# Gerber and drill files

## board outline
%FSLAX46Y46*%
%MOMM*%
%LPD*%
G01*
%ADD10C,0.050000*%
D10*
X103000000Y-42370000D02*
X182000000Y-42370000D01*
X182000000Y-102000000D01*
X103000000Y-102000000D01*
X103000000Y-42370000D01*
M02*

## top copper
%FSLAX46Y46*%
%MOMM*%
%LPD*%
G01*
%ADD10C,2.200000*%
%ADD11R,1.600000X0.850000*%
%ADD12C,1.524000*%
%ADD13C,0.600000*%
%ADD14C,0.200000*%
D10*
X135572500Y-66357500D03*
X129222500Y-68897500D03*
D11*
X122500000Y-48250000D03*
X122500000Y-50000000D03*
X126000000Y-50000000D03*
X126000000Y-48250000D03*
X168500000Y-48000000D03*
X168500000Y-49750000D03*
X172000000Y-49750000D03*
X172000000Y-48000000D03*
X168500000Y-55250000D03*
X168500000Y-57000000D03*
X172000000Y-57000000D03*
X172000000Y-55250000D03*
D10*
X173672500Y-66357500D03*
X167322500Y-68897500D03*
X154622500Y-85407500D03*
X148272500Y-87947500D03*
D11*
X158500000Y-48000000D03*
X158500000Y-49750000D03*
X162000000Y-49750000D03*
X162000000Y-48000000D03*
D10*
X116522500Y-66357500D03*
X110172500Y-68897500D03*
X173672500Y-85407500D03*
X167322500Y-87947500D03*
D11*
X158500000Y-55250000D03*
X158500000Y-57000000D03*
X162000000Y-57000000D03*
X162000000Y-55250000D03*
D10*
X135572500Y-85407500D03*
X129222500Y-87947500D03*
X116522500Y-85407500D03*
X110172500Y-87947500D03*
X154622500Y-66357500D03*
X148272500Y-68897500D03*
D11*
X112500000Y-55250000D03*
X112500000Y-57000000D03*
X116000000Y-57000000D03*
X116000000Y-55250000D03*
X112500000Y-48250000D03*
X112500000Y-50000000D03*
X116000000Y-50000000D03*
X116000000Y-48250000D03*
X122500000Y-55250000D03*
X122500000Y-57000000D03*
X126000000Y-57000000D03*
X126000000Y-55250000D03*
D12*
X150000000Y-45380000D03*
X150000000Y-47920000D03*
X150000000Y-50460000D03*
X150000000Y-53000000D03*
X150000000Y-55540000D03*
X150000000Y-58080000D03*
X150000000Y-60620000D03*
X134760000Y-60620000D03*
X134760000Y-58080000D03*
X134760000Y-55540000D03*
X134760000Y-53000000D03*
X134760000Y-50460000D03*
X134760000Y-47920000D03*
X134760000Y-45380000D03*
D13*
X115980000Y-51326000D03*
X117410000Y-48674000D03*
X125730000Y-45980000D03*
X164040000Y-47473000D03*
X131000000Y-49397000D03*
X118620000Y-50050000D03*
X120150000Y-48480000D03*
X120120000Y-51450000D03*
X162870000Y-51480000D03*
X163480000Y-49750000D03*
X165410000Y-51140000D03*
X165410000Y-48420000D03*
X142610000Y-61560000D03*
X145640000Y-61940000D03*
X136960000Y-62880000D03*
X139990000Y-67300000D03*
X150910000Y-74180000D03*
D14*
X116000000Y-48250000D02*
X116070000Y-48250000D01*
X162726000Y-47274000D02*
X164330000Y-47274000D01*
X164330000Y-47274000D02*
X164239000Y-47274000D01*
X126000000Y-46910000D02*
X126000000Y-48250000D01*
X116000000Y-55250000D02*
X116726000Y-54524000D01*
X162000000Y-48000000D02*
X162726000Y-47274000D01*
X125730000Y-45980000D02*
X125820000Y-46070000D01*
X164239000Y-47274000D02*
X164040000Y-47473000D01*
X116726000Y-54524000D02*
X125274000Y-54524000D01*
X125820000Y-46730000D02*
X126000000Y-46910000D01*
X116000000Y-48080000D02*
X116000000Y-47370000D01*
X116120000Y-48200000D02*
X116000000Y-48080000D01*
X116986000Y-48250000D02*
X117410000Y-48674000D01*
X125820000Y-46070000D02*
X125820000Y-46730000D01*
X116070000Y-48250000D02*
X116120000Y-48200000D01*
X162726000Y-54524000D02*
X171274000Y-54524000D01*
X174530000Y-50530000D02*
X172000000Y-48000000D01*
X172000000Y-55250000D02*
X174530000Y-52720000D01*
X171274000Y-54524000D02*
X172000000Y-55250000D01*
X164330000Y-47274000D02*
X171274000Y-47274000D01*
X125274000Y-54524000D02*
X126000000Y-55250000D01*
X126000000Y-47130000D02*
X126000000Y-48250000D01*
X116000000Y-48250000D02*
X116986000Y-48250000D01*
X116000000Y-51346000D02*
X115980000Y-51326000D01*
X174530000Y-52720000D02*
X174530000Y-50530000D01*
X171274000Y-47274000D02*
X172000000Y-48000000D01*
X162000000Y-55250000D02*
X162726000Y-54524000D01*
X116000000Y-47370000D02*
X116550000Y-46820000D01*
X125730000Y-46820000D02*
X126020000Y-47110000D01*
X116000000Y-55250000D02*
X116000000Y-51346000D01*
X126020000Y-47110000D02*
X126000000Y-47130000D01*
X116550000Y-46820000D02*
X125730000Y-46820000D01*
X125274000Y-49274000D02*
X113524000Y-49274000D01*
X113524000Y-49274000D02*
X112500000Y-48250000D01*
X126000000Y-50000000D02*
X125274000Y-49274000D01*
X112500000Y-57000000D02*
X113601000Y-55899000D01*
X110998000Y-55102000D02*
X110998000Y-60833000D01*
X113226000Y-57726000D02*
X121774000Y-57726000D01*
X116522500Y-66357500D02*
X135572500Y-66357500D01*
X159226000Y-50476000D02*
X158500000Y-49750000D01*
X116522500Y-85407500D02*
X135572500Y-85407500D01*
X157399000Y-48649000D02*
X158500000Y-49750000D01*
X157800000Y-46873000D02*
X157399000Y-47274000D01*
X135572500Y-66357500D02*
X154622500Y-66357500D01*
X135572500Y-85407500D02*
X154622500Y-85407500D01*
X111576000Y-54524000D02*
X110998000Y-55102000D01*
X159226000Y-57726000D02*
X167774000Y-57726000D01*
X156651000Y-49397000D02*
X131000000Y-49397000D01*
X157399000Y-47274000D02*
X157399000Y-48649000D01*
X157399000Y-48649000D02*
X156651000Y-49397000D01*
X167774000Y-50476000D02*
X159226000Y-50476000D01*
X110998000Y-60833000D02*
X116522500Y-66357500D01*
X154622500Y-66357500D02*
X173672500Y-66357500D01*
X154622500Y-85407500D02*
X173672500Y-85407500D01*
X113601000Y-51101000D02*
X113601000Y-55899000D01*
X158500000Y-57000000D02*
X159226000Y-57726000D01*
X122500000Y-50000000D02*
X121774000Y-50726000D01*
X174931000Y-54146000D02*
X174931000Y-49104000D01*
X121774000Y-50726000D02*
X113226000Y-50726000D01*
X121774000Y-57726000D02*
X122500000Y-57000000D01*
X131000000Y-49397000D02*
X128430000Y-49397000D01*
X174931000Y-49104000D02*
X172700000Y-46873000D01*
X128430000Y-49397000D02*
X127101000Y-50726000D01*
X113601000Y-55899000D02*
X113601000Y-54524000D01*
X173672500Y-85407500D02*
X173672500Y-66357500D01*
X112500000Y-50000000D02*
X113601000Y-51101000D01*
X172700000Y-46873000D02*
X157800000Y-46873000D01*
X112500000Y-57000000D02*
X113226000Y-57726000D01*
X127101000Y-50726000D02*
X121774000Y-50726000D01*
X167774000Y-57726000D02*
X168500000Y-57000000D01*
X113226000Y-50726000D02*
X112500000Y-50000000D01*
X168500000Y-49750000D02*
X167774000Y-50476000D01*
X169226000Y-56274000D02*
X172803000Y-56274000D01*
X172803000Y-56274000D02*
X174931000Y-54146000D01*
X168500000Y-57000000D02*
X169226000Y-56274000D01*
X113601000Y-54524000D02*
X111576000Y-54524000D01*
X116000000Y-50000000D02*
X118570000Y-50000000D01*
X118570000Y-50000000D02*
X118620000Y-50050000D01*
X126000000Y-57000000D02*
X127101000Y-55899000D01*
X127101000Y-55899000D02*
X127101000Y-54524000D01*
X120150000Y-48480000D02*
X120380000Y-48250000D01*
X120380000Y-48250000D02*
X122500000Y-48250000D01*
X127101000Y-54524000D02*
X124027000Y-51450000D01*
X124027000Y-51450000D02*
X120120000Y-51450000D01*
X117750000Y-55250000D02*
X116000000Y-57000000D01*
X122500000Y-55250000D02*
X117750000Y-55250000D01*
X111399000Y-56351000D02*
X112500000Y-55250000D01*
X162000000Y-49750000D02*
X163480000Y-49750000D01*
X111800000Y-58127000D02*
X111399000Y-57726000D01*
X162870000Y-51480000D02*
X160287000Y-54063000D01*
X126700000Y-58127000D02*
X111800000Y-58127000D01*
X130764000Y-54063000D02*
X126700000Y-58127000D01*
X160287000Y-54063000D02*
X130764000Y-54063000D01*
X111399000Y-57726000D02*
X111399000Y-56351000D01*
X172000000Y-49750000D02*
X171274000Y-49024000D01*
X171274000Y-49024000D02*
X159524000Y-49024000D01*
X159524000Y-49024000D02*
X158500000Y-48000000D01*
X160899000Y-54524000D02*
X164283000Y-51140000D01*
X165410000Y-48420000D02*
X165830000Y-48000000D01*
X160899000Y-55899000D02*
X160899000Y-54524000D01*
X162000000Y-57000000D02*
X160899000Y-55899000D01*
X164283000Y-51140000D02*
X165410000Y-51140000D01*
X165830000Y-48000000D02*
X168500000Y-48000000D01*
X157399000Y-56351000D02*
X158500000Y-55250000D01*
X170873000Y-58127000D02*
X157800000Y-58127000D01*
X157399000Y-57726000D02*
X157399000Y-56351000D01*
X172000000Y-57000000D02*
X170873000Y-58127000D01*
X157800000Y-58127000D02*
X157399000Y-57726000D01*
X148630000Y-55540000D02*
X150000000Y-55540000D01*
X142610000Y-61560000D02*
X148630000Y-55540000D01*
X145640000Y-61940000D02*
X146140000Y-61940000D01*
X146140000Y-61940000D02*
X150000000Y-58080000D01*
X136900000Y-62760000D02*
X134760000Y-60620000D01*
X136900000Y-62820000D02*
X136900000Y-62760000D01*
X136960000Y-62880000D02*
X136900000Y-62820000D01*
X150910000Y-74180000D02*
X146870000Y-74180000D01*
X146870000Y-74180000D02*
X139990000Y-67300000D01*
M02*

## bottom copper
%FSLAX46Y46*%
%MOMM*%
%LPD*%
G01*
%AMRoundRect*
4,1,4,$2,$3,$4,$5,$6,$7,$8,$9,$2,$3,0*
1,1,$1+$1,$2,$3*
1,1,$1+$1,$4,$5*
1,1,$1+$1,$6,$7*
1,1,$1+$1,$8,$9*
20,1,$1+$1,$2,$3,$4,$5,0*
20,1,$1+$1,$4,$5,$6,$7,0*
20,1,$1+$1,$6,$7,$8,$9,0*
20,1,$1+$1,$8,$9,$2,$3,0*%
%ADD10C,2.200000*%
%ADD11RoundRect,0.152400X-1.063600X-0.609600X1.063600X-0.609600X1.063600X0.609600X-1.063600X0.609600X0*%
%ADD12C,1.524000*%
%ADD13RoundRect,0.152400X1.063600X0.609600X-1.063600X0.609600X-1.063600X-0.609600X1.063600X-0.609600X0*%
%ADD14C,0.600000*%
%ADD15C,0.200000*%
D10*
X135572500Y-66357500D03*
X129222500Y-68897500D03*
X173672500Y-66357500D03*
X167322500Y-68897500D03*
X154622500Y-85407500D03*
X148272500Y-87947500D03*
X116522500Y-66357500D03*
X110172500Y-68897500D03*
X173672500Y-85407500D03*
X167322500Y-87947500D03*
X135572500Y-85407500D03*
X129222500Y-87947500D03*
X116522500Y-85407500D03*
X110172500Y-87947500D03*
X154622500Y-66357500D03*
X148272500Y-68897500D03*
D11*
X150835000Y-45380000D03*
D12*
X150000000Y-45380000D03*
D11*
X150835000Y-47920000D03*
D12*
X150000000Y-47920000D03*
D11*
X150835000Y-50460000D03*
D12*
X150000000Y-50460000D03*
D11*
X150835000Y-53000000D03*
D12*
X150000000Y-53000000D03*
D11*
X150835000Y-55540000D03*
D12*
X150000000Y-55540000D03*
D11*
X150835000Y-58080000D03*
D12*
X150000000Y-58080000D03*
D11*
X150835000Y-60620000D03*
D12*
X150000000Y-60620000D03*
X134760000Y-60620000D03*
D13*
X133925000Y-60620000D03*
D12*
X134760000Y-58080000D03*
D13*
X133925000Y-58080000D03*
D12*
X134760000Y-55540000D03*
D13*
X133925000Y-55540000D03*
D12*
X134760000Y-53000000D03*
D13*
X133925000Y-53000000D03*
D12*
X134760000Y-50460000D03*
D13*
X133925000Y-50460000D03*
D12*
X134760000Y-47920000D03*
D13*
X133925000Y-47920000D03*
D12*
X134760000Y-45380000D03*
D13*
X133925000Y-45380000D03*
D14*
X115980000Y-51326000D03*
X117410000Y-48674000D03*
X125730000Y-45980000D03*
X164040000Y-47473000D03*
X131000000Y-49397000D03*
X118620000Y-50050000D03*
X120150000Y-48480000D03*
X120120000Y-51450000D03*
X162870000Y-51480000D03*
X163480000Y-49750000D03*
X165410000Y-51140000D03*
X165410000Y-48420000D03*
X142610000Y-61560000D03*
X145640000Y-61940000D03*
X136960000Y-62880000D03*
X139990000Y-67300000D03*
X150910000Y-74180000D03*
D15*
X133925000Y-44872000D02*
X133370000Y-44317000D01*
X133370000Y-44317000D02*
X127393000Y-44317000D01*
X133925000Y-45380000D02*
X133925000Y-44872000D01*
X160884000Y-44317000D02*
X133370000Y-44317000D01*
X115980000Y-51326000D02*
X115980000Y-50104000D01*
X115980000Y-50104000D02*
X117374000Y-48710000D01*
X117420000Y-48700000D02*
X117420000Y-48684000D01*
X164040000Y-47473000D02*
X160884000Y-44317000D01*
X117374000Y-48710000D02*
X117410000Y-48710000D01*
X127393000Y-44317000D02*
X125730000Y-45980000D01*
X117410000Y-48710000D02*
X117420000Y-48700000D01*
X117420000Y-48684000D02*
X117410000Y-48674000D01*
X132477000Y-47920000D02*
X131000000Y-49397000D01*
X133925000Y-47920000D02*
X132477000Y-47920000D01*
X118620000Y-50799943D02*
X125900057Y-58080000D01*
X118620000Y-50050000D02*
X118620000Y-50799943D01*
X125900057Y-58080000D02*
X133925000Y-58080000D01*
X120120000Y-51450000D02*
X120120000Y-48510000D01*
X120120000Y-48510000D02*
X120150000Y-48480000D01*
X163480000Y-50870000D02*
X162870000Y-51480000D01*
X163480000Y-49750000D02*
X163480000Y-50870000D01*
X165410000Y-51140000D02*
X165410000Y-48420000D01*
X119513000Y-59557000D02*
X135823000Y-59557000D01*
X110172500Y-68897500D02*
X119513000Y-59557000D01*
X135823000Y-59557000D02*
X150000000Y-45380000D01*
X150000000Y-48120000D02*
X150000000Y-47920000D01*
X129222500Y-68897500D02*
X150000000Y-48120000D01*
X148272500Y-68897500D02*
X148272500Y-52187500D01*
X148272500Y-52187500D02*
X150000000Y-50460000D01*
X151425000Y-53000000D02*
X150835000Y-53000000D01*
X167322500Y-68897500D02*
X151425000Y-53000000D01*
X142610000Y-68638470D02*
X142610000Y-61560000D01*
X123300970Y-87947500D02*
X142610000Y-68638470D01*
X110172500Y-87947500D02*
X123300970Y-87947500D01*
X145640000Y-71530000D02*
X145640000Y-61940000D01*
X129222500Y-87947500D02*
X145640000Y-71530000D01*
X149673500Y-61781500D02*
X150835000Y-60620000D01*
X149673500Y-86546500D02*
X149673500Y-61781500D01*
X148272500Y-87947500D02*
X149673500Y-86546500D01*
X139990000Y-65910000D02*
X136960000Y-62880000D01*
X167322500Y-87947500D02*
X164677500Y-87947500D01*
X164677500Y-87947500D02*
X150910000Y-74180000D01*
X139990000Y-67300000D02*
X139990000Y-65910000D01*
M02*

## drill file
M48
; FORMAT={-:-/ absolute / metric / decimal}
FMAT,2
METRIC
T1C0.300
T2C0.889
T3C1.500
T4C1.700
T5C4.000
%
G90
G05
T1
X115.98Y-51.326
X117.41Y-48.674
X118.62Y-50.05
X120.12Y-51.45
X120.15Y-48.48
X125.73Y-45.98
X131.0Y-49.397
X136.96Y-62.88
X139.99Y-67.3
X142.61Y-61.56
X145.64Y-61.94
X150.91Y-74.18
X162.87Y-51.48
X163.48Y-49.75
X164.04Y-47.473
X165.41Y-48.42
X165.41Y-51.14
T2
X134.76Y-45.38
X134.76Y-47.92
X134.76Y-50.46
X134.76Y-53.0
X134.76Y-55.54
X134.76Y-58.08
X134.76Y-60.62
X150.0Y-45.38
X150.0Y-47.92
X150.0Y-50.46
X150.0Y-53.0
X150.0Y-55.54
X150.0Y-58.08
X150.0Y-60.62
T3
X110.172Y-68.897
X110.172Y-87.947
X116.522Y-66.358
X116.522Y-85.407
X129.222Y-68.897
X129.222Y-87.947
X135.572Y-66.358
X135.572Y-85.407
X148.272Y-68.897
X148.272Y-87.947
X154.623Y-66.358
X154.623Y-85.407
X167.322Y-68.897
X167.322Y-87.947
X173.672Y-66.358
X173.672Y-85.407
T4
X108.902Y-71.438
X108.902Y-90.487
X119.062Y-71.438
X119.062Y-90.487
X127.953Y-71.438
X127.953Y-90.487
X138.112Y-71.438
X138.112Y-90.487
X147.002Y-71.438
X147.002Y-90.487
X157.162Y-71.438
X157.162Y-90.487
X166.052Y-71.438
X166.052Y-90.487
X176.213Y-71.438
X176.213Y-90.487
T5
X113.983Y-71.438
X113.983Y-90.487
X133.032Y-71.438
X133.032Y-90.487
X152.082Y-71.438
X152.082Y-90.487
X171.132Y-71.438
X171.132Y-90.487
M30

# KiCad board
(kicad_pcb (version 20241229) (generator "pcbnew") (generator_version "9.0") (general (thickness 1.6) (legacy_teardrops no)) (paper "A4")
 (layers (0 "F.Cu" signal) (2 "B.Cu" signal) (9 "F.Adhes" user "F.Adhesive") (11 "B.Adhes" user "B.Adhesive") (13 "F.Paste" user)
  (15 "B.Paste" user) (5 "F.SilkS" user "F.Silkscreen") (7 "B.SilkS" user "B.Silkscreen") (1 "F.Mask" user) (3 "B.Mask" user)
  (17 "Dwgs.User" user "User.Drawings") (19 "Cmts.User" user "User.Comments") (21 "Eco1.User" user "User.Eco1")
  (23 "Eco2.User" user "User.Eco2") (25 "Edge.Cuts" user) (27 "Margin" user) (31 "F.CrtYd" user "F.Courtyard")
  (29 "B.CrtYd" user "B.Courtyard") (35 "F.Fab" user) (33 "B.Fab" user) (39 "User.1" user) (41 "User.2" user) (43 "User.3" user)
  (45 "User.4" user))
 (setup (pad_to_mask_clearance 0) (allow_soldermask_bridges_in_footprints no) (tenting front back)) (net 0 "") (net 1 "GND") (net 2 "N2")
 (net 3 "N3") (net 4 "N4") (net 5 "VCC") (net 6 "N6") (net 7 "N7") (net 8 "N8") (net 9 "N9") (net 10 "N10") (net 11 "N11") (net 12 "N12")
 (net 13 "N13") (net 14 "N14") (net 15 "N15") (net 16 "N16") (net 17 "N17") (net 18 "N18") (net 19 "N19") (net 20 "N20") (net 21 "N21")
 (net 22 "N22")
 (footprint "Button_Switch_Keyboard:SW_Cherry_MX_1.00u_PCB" (layer "F.Cu") (at 135.5725 66.3575)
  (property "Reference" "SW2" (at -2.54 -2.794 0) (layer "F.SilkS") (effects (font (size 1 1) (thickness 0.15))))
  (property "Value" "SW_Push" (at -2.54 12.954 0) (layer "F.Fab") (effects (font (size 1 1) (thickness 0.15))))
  (pad "" np_thru_hole circle (at -7.62 5.08) (size 1.7 1.7) (drill 1.7) (layers "*.Cu" "*.Mask"))
  (pad "" np_thru_hole circle (at -2.54 5.08) (size 4 4) (drill 4) (layers "*.Cu" "*.Mask"))
  (pad "" np_thru_hole circle (at 2.54 5.08) (size 1.7 1.7) (drill 1.7) (layers "*.Cu" "*.Mask"))
  (pad "1" thru_hole circle (at 0 0) (size 2.2 2.2) (drill 1.5) (layers "*.Cu" "*.Mask") (remove_unused_layers no) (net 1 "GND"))
  (pad "2" thru_hole circle (at -6.35 2.54) (size 2.2 2.2) (drill 1.5) (layers "*.Cu" "*.Mask") (remove_unused_layers no) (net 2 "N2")))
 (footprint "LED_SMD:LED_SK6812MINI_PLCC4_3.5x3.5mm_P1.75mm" (layer "F.Cu") (at 124.25 49.125)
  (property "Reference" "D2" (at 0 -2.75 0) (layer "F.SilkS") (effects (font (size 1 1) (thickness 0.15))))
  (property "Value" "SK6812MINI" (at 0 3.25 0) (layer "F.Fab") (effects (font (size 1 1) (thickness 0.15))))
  (pad "1" smd rect (at -1.75 -0.875) (size 1.6 0.85) (layers "F.Cu" "F.Mask" "F.Paste") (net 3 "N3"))
  (pad "2" smd rect (at -1.75 0.875) (size 1.6 0.85) (layers "F.Cu" "F.Mask" "F.Paste") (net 1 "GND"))
  (pad "3" smd rect (at 1.75 0.875) (size 1.6 0.85) (layers "F.Cu" "F.Mask" "F.Paste") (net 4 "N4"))
  (pad "4" smd rect (at 1.75 -0.875) (size 1.6 0.85) (layers "F.Cu" "F.Mask" "F.Paste") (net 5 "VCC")))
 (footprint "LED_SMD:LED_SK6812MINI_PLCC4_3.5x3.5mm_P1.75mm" (layer "F.Cu") (at 170.25 48.875)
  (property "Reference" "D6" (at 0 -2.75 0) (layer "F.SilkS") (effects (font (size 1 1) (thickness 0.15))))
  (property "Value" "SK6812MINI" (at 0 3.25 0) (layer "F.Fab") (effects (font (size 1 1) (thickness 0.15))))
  (pad "1" smd rect (at -1.75 -0.875) (size 1.6 0.85) (layers "F.Cu" "F.Mask" "F.Paste") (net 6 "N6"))
  (pad "2" smd rect (at -1.75 0.875) (size 1.6 0.85) (layers "F.Cu" "F.Mask" "F.Paste") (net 1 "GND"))
  (pad "3" smd rect (at 1.75 0.875) (size 1.6 0.85) (layers "F.Cu" "F.Mask" "F.Paste") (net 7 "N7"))
  (pad "4" smd rect (at 1.75 -0.875) (size 1.6 0.85) (layers "F.Cu" "F.Mask" "F.Paste") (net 5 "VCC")))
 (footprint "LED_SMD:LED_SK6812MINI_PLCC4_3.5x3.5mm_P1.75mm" (layer "F.Cu") (at 170.25 56.125)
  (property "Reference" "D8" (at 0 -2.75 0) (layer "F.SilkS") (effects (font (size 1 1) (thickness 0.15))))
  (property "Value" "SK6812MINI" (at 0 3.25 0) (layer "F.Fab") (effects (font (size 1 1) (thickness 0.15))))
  (pad "1" smd rect (at -1.75 -0.875) (size 1.6 0.85) (layers "F.Cu" "F.Mask" "F.Paste") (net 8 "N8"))
  (pad "2" smd rect (at -1.75 0.875) (size 1.6 0.85) (layers "F.Cu" "F.Mask" "F.Paste") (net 1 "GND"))
  (pad "3" smd rect (at 1.75 0.875) (size 1.6 0.85) (layers "F.Cu" "F.Mask" "F.Paste") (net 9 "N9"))
  (pad "4" smd rect (at 1.75 -0.875) (size 1.6 0.85) (layers "F.Cu" "F.Mask" "F.Paste") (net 5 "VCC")))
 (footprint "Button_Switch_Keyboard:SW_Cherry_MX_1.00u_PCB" (layer "F.Cu") (at 173.6725 66.3575)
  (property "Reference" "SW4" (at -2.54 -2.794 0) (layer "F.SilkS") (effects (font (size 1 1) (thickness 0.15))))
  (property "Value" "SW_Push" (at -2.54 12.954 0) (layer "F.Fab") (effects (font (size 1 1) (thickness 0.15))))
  (pad "" np_thru_hole circle (at -7.62 5.08) (size 1.7 1.7) (drill 1.7) (layers "*.Cu" "*.Mask"))
  (pad "" np_thru_hole circle (at -2.54 5.08) (size 4 4) (drill 4) (layers "*.Cu" "*.Mask"))
  (pad "" np_thru_hole circle (at 2.54 5.08) (size 1.7 1.7) (drill 1.7) (layers "*.Cu" "*.Mask"))
  (pad "1" thru_hole circle (at 0 0) (size 2.2 2.2) (drill 1.5) (layers "*.Cu" "*.Mask") (remove_unused_layers no) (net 1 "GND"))
  (pad "2" thru_hole circle (at -6.35 2.54) (size 2.2 2.2) (drill 1.5) (layers "*.Cu" "*.Mask") (remove_unused_layers no) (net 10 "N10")))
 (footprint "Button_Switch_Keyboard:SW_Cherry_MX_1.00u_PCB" (layer "F.Cu") (at 154.6225 85.4075)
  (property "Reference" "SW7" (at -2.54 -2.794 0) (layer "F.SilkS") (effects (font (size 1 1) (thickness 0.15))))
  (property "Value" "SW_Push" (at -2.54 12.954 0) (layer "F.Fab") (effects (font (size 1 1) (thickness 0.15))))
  (pad "" np_thru_hole circle (at -7.62 5.08) (size 1.7 1.7) (drill 1.7) (layers "*.Cu" "*.Mask"))
  (pad "" np_thru_hole circle (at -2.54 5.08) (size 4 4) (drill 4) (layers "*.Cu" "*.Mask"))
  (pad "" np_thru_hole circle (at 2.54 5.08) (size 1.7 1.7) (drill 1.7) (layers "*.Cu" "*.Mask"))
  (pad "1" thru_hole circle (at 0 0) (size 2.2 2.2) (drill 1.5) (layers "*.Cu" "*.Mask") (remove_unused_layers no) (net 1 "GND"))
  (pad "2" thru_hole circle (at -6.35 2.54) (size 2.2 2.2) (drill 1.5) (layers "*.Cu" "*.Mask") (remove_unused_layers no) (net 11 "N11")))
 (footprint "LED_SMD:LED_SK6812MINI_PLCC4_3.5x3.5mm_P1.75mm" (layer "F.Cu") (at 160.25 48.875)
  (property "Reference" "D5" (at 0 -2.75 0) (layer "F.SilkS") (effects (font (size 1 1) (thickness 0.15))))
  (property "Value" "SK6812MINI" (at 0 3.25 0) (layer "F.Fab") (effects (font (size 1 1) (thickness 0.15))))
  (pad "1" smd rect (at -1.75 -0.875) (size 1.6 0.85) (layers "F.Cu" "F.Mask" "F.Paste") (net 7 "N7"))
  (pad "2" smd rect (at -1.75 0.875) (size 1.6 0.85) (layers "F.Cu" "F.Mask" "F.Paste") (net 1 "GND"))
  (pad "3" smd rect (at 1.75 0.875) (size 1.6 0.85) (layers "F.Cu" "F.Mask" "F.Paste") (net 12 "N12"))
  (pad "4" smd rect (at 1.75 -0.875) (size 1.6 0.85) (layers "F.Cu" "F.Mask" "F.Paste") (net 5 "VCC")))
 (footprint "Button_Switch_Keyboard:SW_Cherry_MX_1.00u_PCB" (layer "F.Cu") (at 116.5225 66.3575)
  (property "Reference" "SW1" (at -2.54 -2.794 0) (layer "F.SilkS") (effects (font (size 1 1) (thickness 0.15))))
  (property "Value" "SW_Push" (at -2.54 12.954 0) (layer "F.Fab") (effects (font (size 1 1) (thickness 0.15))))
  (pad "" np_thru_hole circle (at -7.62 5.08) (size 1.7 1.7) (drill 1.7) (layers "*.Cu" "*.Mask"))
  (pad "" np_thru_hole circle (at -2.54 5.08) (size 4 4) (drill 4) (layers "*.Cu" "*.Mask"))
  (pad "" np_thru_hole circle (at 2.54 5.08) (size 1.7 1.7) (drill 1.7) (layers "*.Cu" "*.Mask"))
  (pad "1" thru_hole circle (at 0 0) (size 2.2 2.2) (drill 1.5) (layers "*.Cu" "*.Mask") (remove_unused_layers no) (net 1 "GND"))
  (pad "2" thru_hole circle (at -6.35 2.54) (size 2.2 2.2) (drill 1.5) (layers "*.Cu" "*.Mask") (remove_unused_layers no) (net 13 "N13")))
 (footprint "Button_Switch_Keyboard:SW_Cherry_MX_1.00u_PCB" (layer "F.Cu") (at 173.6725 85.4075)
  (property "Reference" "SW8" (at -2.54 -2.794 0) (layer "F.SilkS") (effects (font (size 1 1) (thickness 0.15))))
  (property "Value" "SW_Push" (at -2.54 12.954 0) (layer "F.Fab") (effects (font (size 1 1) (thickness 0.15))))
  (pad "" np_thru_hole circle (at -7.62 5.08) (size 1.7 1.7) (drill 1.7) (layers "*.Cu" "*.Mask"))
  (pad "" np_thru_hole circle (at -2.54 5.08) (size 4 4) (drill 4) (layers "*.Cu" "*.Mask"))
  (pad "" np_thru_hole circle (at 2.54 5.08) (size 1.7 1.7) (drill 1.7) (layers "*.Cu" "*.Mask"))
  (pad "1" thru_hole circle (at 0 0) (size 2.2 2.2) (drill 1.5) (layers "*.Cu" "*.Mask") (remove_unused_layers no) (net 1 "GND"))
  (pad "2" thru_hole circle (at -6.35 2.54) (size 2.2 2.2) (drill 1.5) (layers "*.Cu" "*.Mask") (remove_unused_layers no) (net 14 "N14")))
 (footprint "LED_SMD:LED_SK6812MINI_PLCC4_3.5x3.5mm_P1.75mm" (layer "F.Cu") (at 160.25 56.125)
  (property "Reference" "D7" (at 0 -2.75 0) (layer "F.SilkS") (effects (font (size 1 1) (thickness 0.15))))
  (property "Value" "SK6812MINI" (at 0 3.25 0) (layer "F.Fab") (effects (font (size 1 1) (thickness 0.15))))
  (pad "1" smd rect (at -1.75 -0.875) (size 1.6 0.85) (layers "F.Cu" "F.Mask" "F.Paste") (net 9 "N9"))
  (pad "2" smd rect (at -1.75 0.875) (size 1.6 0.85) (layers "F.Cu" "F.Mask" "F.Paste") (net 1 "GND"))
  (pad "3" smd rect (at 1.75 0.875) (size 1.6 0.85) (layers "F.Cu" "F.Mask" "F.Paste") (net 6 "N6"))
  (pad "4" smd rect (at 1.75 -0.875) (size 1.6 0.85) (layers "F.Cu" "F.Mask" "F.Paste") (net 5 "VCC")))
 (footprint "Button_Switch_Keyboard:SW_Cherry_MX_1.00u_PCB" (layer "F.Cu") (at 135.5725 85.4075)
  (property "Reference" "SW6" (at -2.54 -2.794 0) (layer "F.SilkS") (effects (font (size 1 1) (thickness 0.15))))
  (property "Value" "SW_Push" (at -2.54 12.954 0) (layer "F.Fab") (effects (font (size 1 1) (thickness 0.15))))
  (pad "" np_thru_hole circle (at -7.62 5.08) (size 1.7 1.7) (drill 1.7) (layers "*.Cu" "*.Mask"))
  (pad "" np_thru_hole circle (at -2.54 5.08) (size 4 4) (drill 4) (layers "*.Cu" "*.Mask"))
  (pad "" np_thru_hole circle (at 2.54 5.08) (size 1.7 1.7) (drill 1.7) (layers "*.Cu" "*.Mask"))
  (pad "1" thru_hole circle (at 0 0) (size 2.2 2.2) (drill 1.5) (layers "*.Cu" "*.Mask") (remove_unused_layers no) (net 1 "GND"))
  (pad "2" thru_hole circle (at -6.35 2.54) (size 2.2 2.2) (drill 1.5) (layers "*.Cu" "*.Mask") (remove_unused_layers no) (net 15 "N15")))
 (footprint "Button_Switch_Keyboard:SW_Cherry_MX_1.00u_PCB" (layer "F.Cu") (at 116.5225 85.4075)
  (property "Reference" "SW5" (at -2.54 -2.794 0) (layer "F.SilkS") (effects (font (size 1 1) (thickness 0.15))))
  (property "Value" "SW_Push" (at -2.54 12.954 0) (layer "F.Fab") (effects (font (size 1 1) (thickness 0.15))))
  (pad "" np_thru_hole circle (at -7.62 5.08) (size 1.7 1.7) (drill 1.7) (layers "*.Cu" "*.Mask"))
  (pad "" np_thru_hole circle (at -2.54 5.08) (size 4 4) (drill 4) (layers "*.Cu" "*.Mask"))
  (pad "" np_thru_hole circle (at 2.54 5.08) (size 1.7 1.7) (drill 1.7) (layers "*.Cu" "*.Mask"))
  (pad "1" thru_hole circle (at 0 0) (size 2.2 2.2) (drill 1.5) (layers "*.Cu" "*.Mask") (remove_unused_layers no) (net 1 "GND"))
  (pad "2" thru_hole circle (at -6.35 2.54) (size 2.2 2.2) (drill 1.5) (layers "*.Cu" "*.Mask") (remove_unused_layers no) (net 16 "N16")))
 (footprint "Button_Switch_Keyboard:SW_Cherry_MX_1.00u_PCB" (layer "F.Cu") (at 154.6225 66.3575)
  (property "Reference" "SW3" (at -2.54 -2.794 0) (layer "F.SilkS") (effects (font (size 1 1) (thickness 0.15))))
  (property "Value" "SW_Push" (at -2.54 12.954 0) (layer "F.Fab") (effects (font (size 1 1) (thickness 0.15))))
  (pad "" np_thru_hole circle (at -7.62 5.08) (size 1.7 1.7) (drill 1.7) (layers "*.Cu" "*.Mask"))
  (pad "" np_thru_hole circle (at -2.54 5.08) (size 4 4) (drill 4) (layers "*.Cu" "*.Mask"))
  (pad "" np_thru_hole circle (at 2.54 5.08) (size 1.7 1.7) (drill 1.7) (layers "*.Cu" "*.Mask"))
  (pad "1" thru_hole circle (at 0 0) (size 2.2 2.2) (drill 1.5) (layers "*.Cu" "*.Mask") (remove_unused_layers no) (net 1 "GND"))
  (pad "2" thru_hole circle (at -6.35 2.54) (size 2.2 2.2) (drill 1.5) (layers "*.Cu" "*.Mask") (remove_unused_layers no) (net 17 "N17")))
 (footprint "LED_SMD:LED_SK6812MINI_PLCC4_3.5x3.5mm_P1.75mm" (layer "F.Cu") (at 114.25 56.125)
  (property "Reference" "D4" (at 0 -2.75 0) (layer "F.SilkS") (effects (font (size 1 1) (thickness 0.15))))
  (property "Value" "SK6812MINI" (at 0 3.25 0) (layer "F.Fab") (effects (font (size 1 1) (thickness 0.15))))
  (pad "1" smd rect (at -1.75 -0.875) (size 1.6 0.85) (layers "F.Cu" "F.Mask" "F.Paste") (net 12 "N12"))
  (pad "2" smd rect (at -1.75 0.875) (size 1.6 0.85) (layers "F.Cu" "F.Mask" "F.Paste") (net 1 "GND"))
  (pad "3" smd rect (at 1.75 0.875) (size 1.6 0.85) (layers "F.Cu" "F.Mask" "F.Paste") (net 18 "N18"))
  (pad "4" smd rect (at 1.75 -0.875) (size 1.6 0.85) (layers "F.Cu" "F.Mask" "F.Paste") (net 5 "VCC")))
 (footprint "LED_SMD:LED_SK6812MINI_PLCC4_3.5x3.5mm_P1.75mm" (layer "F.Cu") (at 114.25 49.125)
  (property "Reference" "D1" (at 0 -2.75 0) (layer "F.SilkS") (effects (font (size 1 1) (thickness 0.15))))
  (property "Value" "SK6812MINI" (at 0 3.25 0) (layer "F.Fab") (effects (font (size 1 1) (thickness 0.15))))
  (pad "1" smd rect (at -1.75 -0.875) (size 1.6 0.85) (layers "F.Cu" "F.Mask" "F.Paste") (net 4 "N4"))
  (pad "2" smd rect (at -1.75 0.875) (size 1.6 0.85) (layers "F.Cu" "F.Mask" "F.Paste") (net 1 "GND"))
  (pad "3" smd rect (at 1.75 0.875) (size 1.6 0.85) (layers "F.Cu" "F.Mask" "F.Paste") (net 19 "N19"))
  (pad "4" smd rect (at 1.75 -0.875) (size 1.6 0.85) (layers "F.Cu" "F.Mask" "F.Paste") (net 5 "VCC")))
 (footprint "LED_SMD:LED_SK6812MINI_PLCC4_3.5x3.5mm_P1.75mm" (layer "F.Cu") (at 124.25 56.125)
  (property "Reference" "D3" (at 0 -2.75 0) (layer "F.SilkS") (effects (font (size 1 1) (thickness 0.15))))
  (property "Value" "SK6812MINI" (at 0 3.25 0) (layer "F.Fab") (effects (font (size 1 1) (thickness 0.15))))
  (pad "1" smd rect (at -1.75 -0.875) (size 1.6 0.85) (layers "F.Cu" "F.Mask" "F.Paste") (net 18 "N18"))
  (pad "2" smd rect (at -1.75 0.875) (size 1.6 0.85) (layers "F.Cu" "F.Mask" "F.Paste") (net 1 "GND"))
  (pad "3" smd rect (at 1.75 0.875) (size 1.6 0.85) (layers "F.Cu" "F.Mask" "F.Paste") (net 3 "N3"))
  (pad "4" smd rect (at 1.75 -0.875) (size 1.6 0.85) (layers "F.Cu" "F.Mask" "F.Paste") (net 5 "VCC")))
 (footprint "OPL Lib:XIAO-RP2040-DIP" (layer "B.Cu") (at 142.38 53 180)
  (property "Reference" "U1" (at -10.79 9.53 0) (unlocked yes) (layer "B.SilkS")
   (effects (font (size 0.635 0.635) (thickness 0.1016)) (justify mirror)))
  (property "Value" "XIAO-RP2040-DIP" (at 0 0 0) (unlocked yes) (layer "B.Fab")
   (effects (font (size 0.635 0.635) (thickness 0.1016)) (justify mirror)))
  (pad "1" smd roundrect (at -8.455 7.62) (size 2.432 1.524) (layers "B.Cu" "B.Mask") (roundrect_rratio 0.1) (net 13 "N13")
   (thermal_bridge_angle 45))
  (pad "1" thru_hole circle (at -7.62 7.62) (size 1.524 1.524) (drill 0.889) (layers "*.Cu" "*.Mask") (remove_unused_layers no)
   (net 13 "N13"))
  (pad "2" smd roundrect (at -8.455 5.08) (size 2.432 1.524) (layers "B.Cu" "B.Mask") (roundrect_rratio 0.1) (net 2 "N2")
   (thermal_bridge_angle 45))
  (pad "2" thru_hole circle (at -7.62 5.08) (size 1.524 1.524) (drill 0.889) (layers "*.Cu" "*.Mask") (remove_unused_layers no) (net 2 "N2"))
  (pad "3" smd roundrect (at -8.455 2.54) (size 2.432 1.524) (layers "B.Cu" "B.Mask") (roundrect_rratio 0.1) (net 17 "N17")
   (thermal_bridge_angle 45))
  (pad "3" thru_hole circle (at -7.62 2.54) (size 1.524 1.524) (drill 0.889) (layers "*.Cu" "*.Mask") (remove_unused_layers no)
   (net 17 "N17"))
  (pad "4" smd roundrect (at -8.455 0) (size 2.432 1.524) (layers "B.Cu" "B.Mask") (roundrect_rratio 0.1) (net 10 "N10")
   (thermal_bridge_angle 45))
  (pad "4" thru_hole circle (at -7.62 0) (size 1.524 1.524) (drill 0.889) (layers "*.Cu" "*.Mask") (remove_unused_layers no) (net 10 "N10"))
  (pad "5" smd roundrect (at -8.455 -2.54) (size 2.432 1.524) (layers "B.Cu" "B.Mask") (roundrect_rratio 0.1) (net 16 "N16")
   (thermal_bridge_angle 45))
  (pad "5" thru_hole circle (at -7.62 -2.54) (size 1.524 1.524) (drill 0.889) (layers "*.Cu" "*.Mask") (remove_unused_layers no)
   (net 16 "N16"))
  (pad "6" smd roundrect (at -8.455 -5.08) (size 2.432 1.524) (layers "B.Cu" "B.Mask") (roundrect_rratio 0.1) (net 15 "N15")
   (thermal_bridge_angle 45))
  (pad "6" thru_hole circle (at -7.62 -5.08) (size 1.524 1.524) (drill 0.889) (layers "*.Cu" "*.Mask") (remove_unused_layers no)
   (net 15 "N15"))
  (pad "7" smd roundrect (at -8.455 -7.62) (size 2.432 1.524) (layers "B.Cu" "B.Mask") (roundrect_rratio 0.1) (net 11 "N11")
   (thermal_bridge_angle 45))
  (pad "7" thru_hole circle (at -7.62 -7.62) (size 1.524 1.524) (drill 0.889) (layers "*.Cu" "*.Mask") (remove_unused_layers no)
   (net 11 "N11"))
  (pad "8" thru_hole circle (at 7.62 -7.62 180) (size 1.524 1.524) (drill 0.889) (layers "*.Cu" "*.Mask") (remove_unused_layers no)
   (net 14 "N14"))
  (pad "8" smd roundrect (at 8.455 -7.62 180) (size 2.432 1.524) (layers "B.Cu" "B.Mask") (roundrect_rratio 0.1) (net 14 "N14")
   (thermal_bridge_angle 45))
  (pad "9" thru_hole circle (at 7.62 -5.08 180) (size 1.524 1.524) (drill 0.889) (layers "*.Cu" "*.Mask") (remove_unused_layers no)
   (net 19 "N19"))
  (pad "9" smd roundrect (at 8.455 -5.08 180) (size 2.432 1.524) (layers "B.Cu" "B.Mask") (roundrect_rratio 0.1) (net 19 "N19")
   (thermal_bridge_angle 45))
  (pad "10" thru_hole circle (at 7.62 -2.54 180) (size 1.524 1.524) (drill 0.889) (layers "*.Cu" "*.Mask") (remove_unused_layers no)
   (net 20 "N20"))
  (pad "10" smd roundrect (at 8.455 -2.54 180) (size 2.432 1.524) (layers "B.Cu" "B.Mask") (roundrect_rratio 0.1) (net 20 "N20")
   (thermal_bridge_angle 45))
  (pad "11" thru_hole circle (at 7.62 0 180) (size 1.524 1.524) (drill 0.889) (layers "*.Cu" "*.Mask") (remove_unused_layers no)
   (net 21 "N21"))
  (pad "11" smd roundrect (at 8.455 0 180) (size 2.432 1.524) (layers "B.Cu" "B.Mask") (roundrect_rratio 0.1) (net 21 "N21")
   (thermal_bridge_angle 45))
  (pad "12" thru_hole circle (at 7.62 2.54 180) (size 1.524 1.524) (drill 0.889) (layers "*.Cu" "*.Mask") (remove_unused_layers no)
   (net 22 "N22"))
  (pad "12" smd roundrect (at 8.455 2.54 180) (size 2.432 1.524) (layers "B.Cu" "B.Mask") (roundrect_rratio 0.1) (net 22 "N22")
   (thermal_bridge_angle 45))
  (pad "13" thru_hole circle (at 7.62 5.08 180) (size 1.524 1.524) (drill 0.889) (layers "*.Cu" "*.Mask") (remove_unused_layers no)
   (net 1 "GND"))
  (pad "13" smd roundrect (at 8.455 5.08 180) (size 2.432 1.524) (layers "B.Cu" "B.Mask") (roundrect_rratio 0.1) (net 1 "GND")
   (thermal_bridge_angle 45))
  (pad "14" thru_hole circle (at 7.62 7.62 180) (size 1.524 1.524) (drill 0.889) (layers "*.Cu" "*.Mask") (remove_unused_layers no)
   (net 5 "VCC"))
  (pad "14" smd roundrect (at 8.455 7.62 180) (size 2.432 1.524) (layers "B.Cu" "B.Mask") (roundrect_rratio 0.1) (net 5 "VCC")
   (thermal_bridge_angle 45)))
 (gr_rect (start 103 42.37) (end 182 102) (stroke (width 0.05) (type default)) (fill no) (layer "Edge.Cuts"))
 (segment (start 116 48.25) (end 116.07 48.25) (width 0.2) (layer "F.Cu") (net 5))
 (segment (start 162.726 47.274) (end 164.33 47.274) (width 0.2) (layer "F.Cu") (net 5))
 (segment (start 164.33 47.274) (end 164.239 47.274) (width 0.2) (layer "F.Cu") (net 5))
 (segment (start 126 46.91) (end 126 48.25) (width 0.2) (layer "F.Cu") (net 5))
 (segment (start 116 55.25) (end 116.726 54.524) (width 0.2) (layer "F.Cu") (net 5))
 (segment (start 162 48) (end 162.726 47.274) (width 0.2) (layer "F.Cu") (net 5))
 (segment (start 125.73 45.98) (end 125.82 46.07) (width 0.2) (layer "F.Cu") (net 5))
 (segment (start 164.239 47.274) (end 164.04 47.473) (width 0.2) (layer "F.Cu") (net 5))
 (segment (start 116.726 54.524) (end 125.274 54.524) (width 0.2) (layer "F.Cu") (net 5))
 (segment (start 125.82 46.73) (end 126 46.91) (width 0.2) (layer "F.Cu") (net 5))
 (segment (start 116 48.08) (end 116 47.37) (width 0.2) (layer "F.Cu") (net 5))
 (segment (start 116.12 48.2) (end 116 48.08) (width 0.2) (layer "F.Cu") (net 5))
 (segment (start 116.986 48.25) (end 117.41 48.674) (width 0.2) (layer "F.Cu") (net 5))
 (segment (start 125.82 46.07) (end 125.82 46.73) (width 0.2) (layer "F.Cu") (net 5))
 (segment (start 116.07 48.25) (end 116.12 48.2) (width 0.2) (layer "F.Cu") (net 5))
 (segment (start 162.726 54.524) (end 171.274 54.524) (width 0.2) (layer "F.Cu") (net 5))
 (segment (start 174.53 50.53) (end 172 48) (width 0.2) (layer "F.Cu") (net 5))
 (segment (start 172 55.25) (end 174.53 52.72) (width 0.2) (layer "F.Cu") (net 5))
 (segment (start 171.274 54.524) (end 172 55.25) (width 0.2) (layer "F.Cu") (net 5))
 (segment (start 164.33 47.274) (end 171.274 47.274) (width 0.2) (layer "F.Cu") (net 5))
 (segment (start 125.274 54.524) (end 126 55.25) (width 0.2) (layer "F.Cu") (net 5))
 (segment (start 126 47.13) (end 126 48.25) (width 0.2) (layer "F.Cu") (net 5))
 (segment (start 116 48.25) (end 116.986 48.25) (width 0.2) (layer "F.Cu") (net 5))
 (segment (start 116 51.346) (end 115.98 51.326) (width 0.2) (layer "F.Cu") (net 5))
 (segment (start 174.53 52.72) (end 174.53 50.53) (width 0.2) (layer "F.Cu") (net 5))
 (segment (start 171.274 47.274) (end 172 48) (width 0.2) (layer "F.Cu") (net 5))
 (segment (start 162 55.25) (end 162.726 54.524) (width 0.2) (layer "F.Cu") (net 5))
 (segment (start 116 47.37) (end 116.55 46.82) (width 0.2) (layer "F.Cu") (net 5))
 (segment (start 125.73 46.82) (end 126.02 47.11) (width 0.2) (layer "F.Cu") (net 5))
 (segment (start 116 55.25) (end 116 51.346) (width 0.2) (layer "F.Cu") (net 5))
 (segment (start 126.02 47.11) (end 126 47.13) (width 0.2) (layer "F.Cu") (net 5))
 (segment (start 116.55 46.82) (end 125.73 46.82) (width 0.2) (layer "F.Cu") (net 5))
 (via (at 115.98 51.326) (size 0.6) (drill 0.3) (layers "F.Cu" "B.Cu") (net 5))
 (via (at 117.41 48.674) (size 0.6) (drill 0.3) (layers "F.Cu" "B.Cu") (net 5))
 (via (at 125.73 45.98) (size 0.6) (drill 0.3) (layers "F.Cu" "B.Cu") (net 5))
 (via (at 164.04 47.473) (size 0.6) (drill 0.3) (layers "F.Cu" "B.Cu") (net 5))
 (segment (start 133.925 44.872) (end 133.37 44.317) (width 0.2) (layer "B.Cu") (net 5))
 (segment (start 133.37 44.317) (end 127.393 44.317) (width 0.2) (layer "B.Cu") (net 5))
 (segment (start 133.925 45.38) (end 133.925 44.872) (width 0.2) (layer "B.Cu") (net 5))
 (segment (start 160.884 44.317) (end 133.37 44.317) (width 0.2) (layer "B.Cu") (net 5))
 (segment (start 115.98 51.326) (end 115.98 50.104) (width 0.2) (layer "B.Cu") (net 5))
 (segment (start 115.98 50.104) (end 117.374 48.71) (width 0.2) (layer "B.Cu") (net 5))
 (segment (start 117.42 48.7) (end 117.42 48.684) (width 0.2) (layer "B.Cu") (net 5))
 (segment (start 164.04 47.473) (end 160.884 44.317) (width 0.2) (layer "B.Cu") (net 5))
 (segment (start 117.374 48.71) (end 117.41 48.71) (width 0.2) (layer "B.Cu") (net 5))
 (segment (start 127.393 44.317) (end 125.73 45.98) (width 0.2) (layer "B.Cu") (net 5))
 (segment (start 117.41 48.71) (end 117.42 48.7) (width 0.2) (layer "B.Cu") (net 5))
 (segment (start 117.42 48.684) (end 117.41 48.674) (width 0.2) (layer "B.Cu") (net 5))
 (segment (start 125.274 49.274) (end 113.524 49.274) (width 0.2) (layer "F.Cu") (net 4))
 (segment (start 113.524 49.274) (end 112.5 48.25) (width 0.2) (layer "F.Cu") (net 4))
 (segment (start 126 50) (end 125.274 49.274) (width 0.2) (layer "F.Cu") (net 4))
 (segment (start 112.5 57) (end 113.601 55.899) (width 0.2) (layer "F.Cu") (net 1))
 (segment (start 110.998 55.102) (end 110.998 60.833) (width 0.2) (layer "F.Cu") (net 1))
 (segment (start 113.226 57.726) (end 121.774 57.726) (width 0.2) (layer "F.Cu") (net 1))
 (segment (start 116.5225 66.3575) (end 135.5725 66.3575) (width 0.2) (layer "F.Cu") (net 1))
 (segment (start 159.226 50.476) (end 158.5 49.75) (width 0.2) (layer "F.Cu") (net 1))
 (segment (start 116.5225 85.4075) (end 135.5725 85.4075) (width 0.2) (layer "F.Cu") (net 1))
 (segment (start 157.399 48.649) (end 158.5 49.75) (width 0.2) (layer "F.Cu") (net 1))
 (segment (start 157.8 46.873) (end 157.399 47.274) (width 0.2) (layer "F.Cu") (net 1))
 (segment (start 135.5725 66.3575) (end 154.6225 66.3575) (width 0.2) (layer "F.Cu") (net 1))
 (segment (start 135.5725 85.4075) (end 154.6225 85.4075) (width 0.2) (layer "F.Cu") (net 1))
 (segment (start 111.576 54.524) (end 110.998 55.102) (width 0.2) (layer "F.Cu") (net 1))
 (segment (start 159.226 57.726) (end 167.774 57.726) (width 0.2) (layer "F.Cu") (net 1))
 (segment (start 156.651 49.397) (end 131 49.397) (width 0.2) (layer "F.Cu") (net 1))
 (segment (start 157.399 47.274) (end 157.399 48.649) (width 0.2) (layer "F.Cu") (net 1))
 (segment (start 157.399 48.649) (end 156.651 49.397) (width 0.2) (layer "F.Cu") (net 1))
 (segment (start 167.774 50.476) (end 159.226 50.476) (width 0.2) (layer "F.Cu") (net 1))
 (segment (start 110.998 60.833) (end 116.5225 66.3575) (width 0.2) (layer "F.Cu") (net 1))
 (segment (start 154.6225 66.3575) (end 173.6725 66.3575) (width 0.2) (layer "F.Cu") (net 1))
 (segment (start 154.6225 85.4075) (end 173.6725 85.4075) (width 0.2) (layer "F.Cu") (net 1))
 (segment (start 113.601 51.101) (end 113.601 55.899) (width 0.2) (layer "F.Cu") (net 1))
 (segment (start 158.5 57) (end 159.226 57.726) (width 0.2) (layer "F.Cu") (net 1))
 (segment (start 122.5 50) (end 121.774 50.726) (width 0.2) (layer "F.Cu") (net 1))
 (segment (start 174.931 54.146) (end 174.931 49.104) (width 0.2) (layer "F.Cu") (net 1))
 (segment (start 121.774 50.726) (end 113.226 50.726) (width 0.2) (layer "F.Cu") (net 1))
 (segment (start 121.774 57.726) (end 122.5 57) (width 0.2) (layer "F.Cu") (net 1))
 (segment (start 131 49.397) (end 128.43 49.397) (width 0.2) (layer "F.Cu") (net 1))
 (segment (start 174.931 49.104) (end 172.7 46.873) (width 0.2) (layer "F.Cu") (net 1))
 (segment (start 128.43 49.397) (end 127.101 50.726) (width 0.2) (layer "F.Cu") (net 1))
 (segment (start 113.601 55.899) (end 113.601 54.524) (width 0.2) (layer "F.Cu") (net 1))
 (segment (start 173.6725 85.4075) (end 173.6725 66.3575) (width 0.2) (layer "F.Cu") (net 1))
 (segment (start 112.5 50) (end 113.601 51.101) (width 0.2) (layer "F.Cu") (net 1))
 (segment (start 172.7 46.873) (end 157.8 46.873) (width 0.2) (layer "F.Cu") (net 1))
 (segment (start 112.5 57) (end 113.226 57.726) (width 0.2) (layer "F.Cu") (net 1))
 (segment (start 127.101 50.726) (end 121.774 50.726) (width 0.2) (layer "F.Cu") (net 1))
 (segment (start 167.774 57.726) (end 168.5 57) (width 0.2) (layer "F.Cu") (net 1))
 (segment (start 113.226 50.726) (end 112.5 50) (width 0.2) (layer "F.Cu") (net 1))
 (segment (start 168.5 49.75) (end 167.774 50.476) (width 0.2) (layer "F.Cu") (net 1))
 (segment (start 169.226 56.274) (end 172.803 56.274) (width 0.2) (layer "F.Cu") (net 1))
 (segment (start 172.803 56.274) (end 174.931 54.146) (width 0.2) (layer "F.Cu") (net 1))
 (segment (start 168.5 57) (end 169.226 56.274) (width 0.2) (layer "F.Cu") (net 1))
 (segment (start 113.601 54.524) (end 111.576 54.524) (width 0.2) (layer "F.Cu") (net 1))
 (via (at 131 49.397) (size 0.6) (drill 0.3) (layers "F.Cu" "B.Cu") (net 1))
 (segment (start 132.477 47.92) (end 131 49.397) (width 0.2) (layer "B.Cu") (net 1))
 (segment (start 133.925 47.92) (end 132.477 47.92) (width 0.2) (layer "B.Cu") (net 1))
 (segment (start 116 50) (end 118.57 50) (width 0.2) (layer "F.Cu") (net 19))
 (segment (start 118.57 50) (end 118.62 50.05) (width 0.2) (layer "F.Cu") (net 19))
 (via (at 118.62 50.05) (size 0.6) (drill 0.3) (layers "F.Cu" "B.Cu") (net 19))
 (segment (start 118.62 50.799943) (end 125.900057 58.08) (width 0.2) (layer "B.Cu") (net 19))
 (segment (start 118.62 50.05) (end 118.62 50.799943) (width 0.2) (layer "B.Cu") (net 19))
 (segment (start 125.900057 58.08) (end 133.925 58.08) (width 0.2) (layer "B.Cu") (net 19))
 (segment (start 126 57) (end 127.101 55.899) (width 0.2) (layer "F.Cu") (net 3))
 (segment (start 127.101 55.899) (end 127.101 54.524) (width 0.2) (layer "F.Cu") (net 3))
 (segment (start 120.15 48.48) (end 120.38 48.25) (width 0.2) (layer "F.Cu") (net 3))
 (segment (start 120.38 48.25) (end 122.5 48.25) (width 0.2) (layer "F.Cu") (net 3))
 (segment (start 127.101 54.524) (end 124.027 51.45) (width 0.2) (layer "F.Cu") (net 3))
 (segment (start 124.027 51.45) (end 120.12 51.45) (width 0.2) (layer "F.Cu") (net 3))
 (via (at 120.15 48.48) (size 0.6) (drill 0.3) (layers "F.Cu" "B.Cu") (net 3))
 (via (at 120.12 51.45) (size 0.6) (drill 0.3) (layers "F.Cu" "B.Cu") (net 3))
 (segment (start 120.12 51.45) (end 120.12 48.51) (width 0.2) (layer "B.Cu") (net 3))
 (segment (start 120.12 48.51) (end 120.15 48.48) (width 0.2) (layer "B.Cu") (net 3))
 (segment (start 117.75 55.25) (end 116 57) (width 0.2) (layer "F.Cu") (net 18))
 (segment (start 122.5 55.25) (end 117.75 55.25) (width 0.2) (layer "F.Cu") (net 18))
 (segment (start 111.399 56.351) (end 112.5 55.25) (width 0.2) (layer "F.Cu") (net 12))
 (segment (start 162 49.75) (end 163.48 49.75) (width 0.2) (layer "F.Cu") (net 12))
 (segment (start 111.8 58.127) (end 111.399 57.726) (width 0.2) (layer "F.Cu") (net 12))
 (segment (start 162.87 51.48) (end 160.287 54.063) (width 0.2) (layer "F.Cu") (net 12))
 (segment (start 126.7 58.127) (end 111.8 58.127) (width 0.2) (layer "F.Cu") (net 12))
 (segment (start 130.764 54.063) (end 126.7 58.127) (width 0.2) (layer "F.Cu") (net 12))
 (segment (start 160.287 54.063) (end 130.764 54.063) (width 0.2) (layer "F.Cu") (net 12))
 (segment (start 111.399 57.726) (end 111.399 56.351) (width 0.2) (layer "F.Cu") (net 12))
 (via (at 162.87 51.48) (size 0.6) (drill 0.3) (layers "F.Cu" "B.Cu") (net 12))
 (via (at 163.48 49.75) (size 0.6) (drill 0.3) (layers "F.Cu" "B.Cu") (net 12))
 (segment (start 163.48 50.87) (end 162.87 51.48) (width 0.2) (layer "B.Cu") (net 12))
 (segment (start 163.48 49.75) (end 163.48 50.87) (width 0.2) (layer "B.Cu") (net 12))
 (segment (start 172 49.75) (end 171.274 49.024) (width 0.2) (layer "F.Cu") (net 7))
 (segment (start 171.274 49.024) (end 159.524 49.024) (width 0.2) (layer "F.Cu") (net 7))
 (segment (start 159.524 49.024) (end 158.5 48) (width 0.2) (layer "F.Cu") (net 7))
 (segment (start 160.899 54.524) (end 164.283 51.14) (width 0.2) (layer "F.Cu") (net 6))
 (segment (start 165.41 48.42) (end 165.83 48) (width 0.2) (layer "F.Cu") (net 6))
 (segment (start 160.899 55.899) (end 160.899 54.524) (width 0.2) (layer "F.Cu") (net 6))
 (segment (start 162 57) (end 160.899 55.899) (width 0.2) (layer "F.Cu") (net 6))
 (segment (start 164.283 51.14) (end 165.41 51.14) (width 0.2) (layer "F.Cu") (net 6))
 (segment (start 165.83 48) (end 168.5 48) (width 0.2) (layer "F.Cu") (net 6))
 (via (at 165.41 51.14) (size 0.6) (drill 0.3) (layers "F.Cu" "B.Cu") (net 6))
 (via (at 165.41 48.42) (size 0.6) (drill 0.3) (layers "F.Cu" "B.Cu") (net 6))
 (segment (start 165.41 51.14) (end 165.41 48.42) (width 0.2) (layer "B.Cu") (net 6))
 (segment (start 157.399 56.351) (end 158.5 55.25) (width 0.2) (layer "F.Cu") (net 9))
 (segment (start 170.873 58.127) (end 157.8 58.127) (width 0.2) (layer "F.Cu") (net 9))
 (segment (start 157.399 57.726) (end 157.399 56.351) (width 0.2) (layer "F.Cu") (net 9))
 (segment (start 172 57) (end 170.873 58.127) (width 0.2) (layer "F.Cu") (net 9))
 (segment (start 157.8 58.127) (end 157.399 57.726) (width 0.2) (layer "F.Cu") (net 9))
 (segment (start 119.513 59.557) (end 135.823 59.557) (width 0.2) (layer "B.Cu") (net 13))
 (segment (start 110.1725 68.8975) (end 119.513 59.557) (width 0.2) (layer "B.Cu") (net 13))
 (segment (start 135.823 59.557) (end 150 45.38) (width 0.2) (layer "B.Cu") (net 13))
 (segment (start 150 48.12) (end 150 47.92) (width 0.2) (layer "B.Cu") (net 2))
 (segment (start 129.2225 68.8975) (end 150 48.12) (width 0.2) (layer "B.Cu") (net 2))
 (segment (start 148.2725 68.8975) (end 148.2725 52.1875) (width 0.2) (layer "B.Cu") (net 17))
 (segment (start 148.2725 52.1875) (end 150 50.46) (width 0.2) (layer "B.Cu") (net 17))
 (segment (start 151.425 53) (end 150.835 53) (width 0.2) (layer "B.Cu") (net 10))
 (segment (start 167.3225 68.8975) (end 151.425 53) (width 0.2) (layer "B.Cu") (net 10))
 (segment (start 148.63 55.54) (end 150 55.54) (width 0.2) (layer "F.Cu") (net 16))
 (segment (start 142.61 61.56) (end 148.63 55.54) (width 0.2) (layer "F.Cu") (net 16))
 (via (at 142.61 61.56) (size 0.6) (drill 0.3) (layers "F.Cu" "B.Cu") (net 16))
 (segment (start 142.61 68.63847) (end 142.61 61.56) (width 0.2) (layer "B.Cu") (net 16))
 (segment (start 123.30097 87.9475) (end 142.61 68.63847) (width 0.2) (layer "B.Cu") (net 16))
 (segment (start 110.1725 87.9475) (end 123.30097 87.9475) (width 0.2) (layer "B.Cu") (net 16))
 (segment (start 145.64 61.94) (end 146.14 61.94) (width 0.2) (layer "F.Cu") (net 15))
 (segment (start 146.14 61.94) (end 150 58.08) (width 0.2) (layer "F.Cu") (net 15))
 (via (at 145.64 61.94) (size 0.6) (drill 0.3) (layers "F.Cu" "B.Cu") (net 15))
 (segment (start 145.64 71.53) (end 145.64 61.94) (width 0.2) (layer "B.Cu") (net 15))
 (segment (start 129.2225 87.9475) (end 145.64 71.53) (width 0.2) (layer "B.Cu") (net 15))
 (segment (start 149.6735 61.7815) (end 150.835 60.62) (width 0.2) (layer "B.Cu") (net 11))
 (segment (start 149.6735 86.5465) (end 149.6735 61.7815) (width 0.2) (layer "B.Cu") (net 11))
 (segment (start 148.2725 87.9475) (end 149.6735 86.5465) (width 0.2) (layer "B.Cu") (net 11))
 (segment (start 136.9 62.76) (end 134.76 60.62) (width 0.2) (layer "F.Cu") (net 14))
 (segment (start 136.9 62.82) (end 136.9 62.76) (width 0.2) (layer "F.Cu") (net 14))
 (segment (start 136.96 62.88) (end 136.9 62.82) (width 0.2) (layer "F.Cu") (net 14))
 (segment (start 150.91 74.18) (end 146.87 74.18) (width 0.2) (layer "F.Cu") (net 14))
 (segment (start 146.87 74.18) (end 139.99 67.3) (width 0.2) (layer "F.Cu") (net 14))
 (via (at 136.96 62.88) (size 0.6) (drill 0.3) (layers "F.Cu" "B.Cu") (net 14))
 (via (at 139.99 67.3) (size 0.6) (drill 0.3) (layers "F.Cu" "B.Cu") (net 14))
 (via (at 150.91 74.18) (size 0.6) (drill 0.3) (layers "F.Cu" "B.Cu") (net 14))
 (segment (start 139.99 65.91) (end 136.96 62.88) (width 0.2) (layer "B.Cu") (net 14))
 (segment (start 167.3225 87.9475) (end 164.6775 87.9475) (width 0.2) (layer "B.Cu") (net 14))
 (segment (start 164.6775 87.9475) (end 150.91 74.18) (width 0.2) (layer "B.Cu") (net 14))
 (segment (start 139.99 67.3) (end 139.99 65.91) (width 0.2) (layer "B.Cu") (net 14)))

